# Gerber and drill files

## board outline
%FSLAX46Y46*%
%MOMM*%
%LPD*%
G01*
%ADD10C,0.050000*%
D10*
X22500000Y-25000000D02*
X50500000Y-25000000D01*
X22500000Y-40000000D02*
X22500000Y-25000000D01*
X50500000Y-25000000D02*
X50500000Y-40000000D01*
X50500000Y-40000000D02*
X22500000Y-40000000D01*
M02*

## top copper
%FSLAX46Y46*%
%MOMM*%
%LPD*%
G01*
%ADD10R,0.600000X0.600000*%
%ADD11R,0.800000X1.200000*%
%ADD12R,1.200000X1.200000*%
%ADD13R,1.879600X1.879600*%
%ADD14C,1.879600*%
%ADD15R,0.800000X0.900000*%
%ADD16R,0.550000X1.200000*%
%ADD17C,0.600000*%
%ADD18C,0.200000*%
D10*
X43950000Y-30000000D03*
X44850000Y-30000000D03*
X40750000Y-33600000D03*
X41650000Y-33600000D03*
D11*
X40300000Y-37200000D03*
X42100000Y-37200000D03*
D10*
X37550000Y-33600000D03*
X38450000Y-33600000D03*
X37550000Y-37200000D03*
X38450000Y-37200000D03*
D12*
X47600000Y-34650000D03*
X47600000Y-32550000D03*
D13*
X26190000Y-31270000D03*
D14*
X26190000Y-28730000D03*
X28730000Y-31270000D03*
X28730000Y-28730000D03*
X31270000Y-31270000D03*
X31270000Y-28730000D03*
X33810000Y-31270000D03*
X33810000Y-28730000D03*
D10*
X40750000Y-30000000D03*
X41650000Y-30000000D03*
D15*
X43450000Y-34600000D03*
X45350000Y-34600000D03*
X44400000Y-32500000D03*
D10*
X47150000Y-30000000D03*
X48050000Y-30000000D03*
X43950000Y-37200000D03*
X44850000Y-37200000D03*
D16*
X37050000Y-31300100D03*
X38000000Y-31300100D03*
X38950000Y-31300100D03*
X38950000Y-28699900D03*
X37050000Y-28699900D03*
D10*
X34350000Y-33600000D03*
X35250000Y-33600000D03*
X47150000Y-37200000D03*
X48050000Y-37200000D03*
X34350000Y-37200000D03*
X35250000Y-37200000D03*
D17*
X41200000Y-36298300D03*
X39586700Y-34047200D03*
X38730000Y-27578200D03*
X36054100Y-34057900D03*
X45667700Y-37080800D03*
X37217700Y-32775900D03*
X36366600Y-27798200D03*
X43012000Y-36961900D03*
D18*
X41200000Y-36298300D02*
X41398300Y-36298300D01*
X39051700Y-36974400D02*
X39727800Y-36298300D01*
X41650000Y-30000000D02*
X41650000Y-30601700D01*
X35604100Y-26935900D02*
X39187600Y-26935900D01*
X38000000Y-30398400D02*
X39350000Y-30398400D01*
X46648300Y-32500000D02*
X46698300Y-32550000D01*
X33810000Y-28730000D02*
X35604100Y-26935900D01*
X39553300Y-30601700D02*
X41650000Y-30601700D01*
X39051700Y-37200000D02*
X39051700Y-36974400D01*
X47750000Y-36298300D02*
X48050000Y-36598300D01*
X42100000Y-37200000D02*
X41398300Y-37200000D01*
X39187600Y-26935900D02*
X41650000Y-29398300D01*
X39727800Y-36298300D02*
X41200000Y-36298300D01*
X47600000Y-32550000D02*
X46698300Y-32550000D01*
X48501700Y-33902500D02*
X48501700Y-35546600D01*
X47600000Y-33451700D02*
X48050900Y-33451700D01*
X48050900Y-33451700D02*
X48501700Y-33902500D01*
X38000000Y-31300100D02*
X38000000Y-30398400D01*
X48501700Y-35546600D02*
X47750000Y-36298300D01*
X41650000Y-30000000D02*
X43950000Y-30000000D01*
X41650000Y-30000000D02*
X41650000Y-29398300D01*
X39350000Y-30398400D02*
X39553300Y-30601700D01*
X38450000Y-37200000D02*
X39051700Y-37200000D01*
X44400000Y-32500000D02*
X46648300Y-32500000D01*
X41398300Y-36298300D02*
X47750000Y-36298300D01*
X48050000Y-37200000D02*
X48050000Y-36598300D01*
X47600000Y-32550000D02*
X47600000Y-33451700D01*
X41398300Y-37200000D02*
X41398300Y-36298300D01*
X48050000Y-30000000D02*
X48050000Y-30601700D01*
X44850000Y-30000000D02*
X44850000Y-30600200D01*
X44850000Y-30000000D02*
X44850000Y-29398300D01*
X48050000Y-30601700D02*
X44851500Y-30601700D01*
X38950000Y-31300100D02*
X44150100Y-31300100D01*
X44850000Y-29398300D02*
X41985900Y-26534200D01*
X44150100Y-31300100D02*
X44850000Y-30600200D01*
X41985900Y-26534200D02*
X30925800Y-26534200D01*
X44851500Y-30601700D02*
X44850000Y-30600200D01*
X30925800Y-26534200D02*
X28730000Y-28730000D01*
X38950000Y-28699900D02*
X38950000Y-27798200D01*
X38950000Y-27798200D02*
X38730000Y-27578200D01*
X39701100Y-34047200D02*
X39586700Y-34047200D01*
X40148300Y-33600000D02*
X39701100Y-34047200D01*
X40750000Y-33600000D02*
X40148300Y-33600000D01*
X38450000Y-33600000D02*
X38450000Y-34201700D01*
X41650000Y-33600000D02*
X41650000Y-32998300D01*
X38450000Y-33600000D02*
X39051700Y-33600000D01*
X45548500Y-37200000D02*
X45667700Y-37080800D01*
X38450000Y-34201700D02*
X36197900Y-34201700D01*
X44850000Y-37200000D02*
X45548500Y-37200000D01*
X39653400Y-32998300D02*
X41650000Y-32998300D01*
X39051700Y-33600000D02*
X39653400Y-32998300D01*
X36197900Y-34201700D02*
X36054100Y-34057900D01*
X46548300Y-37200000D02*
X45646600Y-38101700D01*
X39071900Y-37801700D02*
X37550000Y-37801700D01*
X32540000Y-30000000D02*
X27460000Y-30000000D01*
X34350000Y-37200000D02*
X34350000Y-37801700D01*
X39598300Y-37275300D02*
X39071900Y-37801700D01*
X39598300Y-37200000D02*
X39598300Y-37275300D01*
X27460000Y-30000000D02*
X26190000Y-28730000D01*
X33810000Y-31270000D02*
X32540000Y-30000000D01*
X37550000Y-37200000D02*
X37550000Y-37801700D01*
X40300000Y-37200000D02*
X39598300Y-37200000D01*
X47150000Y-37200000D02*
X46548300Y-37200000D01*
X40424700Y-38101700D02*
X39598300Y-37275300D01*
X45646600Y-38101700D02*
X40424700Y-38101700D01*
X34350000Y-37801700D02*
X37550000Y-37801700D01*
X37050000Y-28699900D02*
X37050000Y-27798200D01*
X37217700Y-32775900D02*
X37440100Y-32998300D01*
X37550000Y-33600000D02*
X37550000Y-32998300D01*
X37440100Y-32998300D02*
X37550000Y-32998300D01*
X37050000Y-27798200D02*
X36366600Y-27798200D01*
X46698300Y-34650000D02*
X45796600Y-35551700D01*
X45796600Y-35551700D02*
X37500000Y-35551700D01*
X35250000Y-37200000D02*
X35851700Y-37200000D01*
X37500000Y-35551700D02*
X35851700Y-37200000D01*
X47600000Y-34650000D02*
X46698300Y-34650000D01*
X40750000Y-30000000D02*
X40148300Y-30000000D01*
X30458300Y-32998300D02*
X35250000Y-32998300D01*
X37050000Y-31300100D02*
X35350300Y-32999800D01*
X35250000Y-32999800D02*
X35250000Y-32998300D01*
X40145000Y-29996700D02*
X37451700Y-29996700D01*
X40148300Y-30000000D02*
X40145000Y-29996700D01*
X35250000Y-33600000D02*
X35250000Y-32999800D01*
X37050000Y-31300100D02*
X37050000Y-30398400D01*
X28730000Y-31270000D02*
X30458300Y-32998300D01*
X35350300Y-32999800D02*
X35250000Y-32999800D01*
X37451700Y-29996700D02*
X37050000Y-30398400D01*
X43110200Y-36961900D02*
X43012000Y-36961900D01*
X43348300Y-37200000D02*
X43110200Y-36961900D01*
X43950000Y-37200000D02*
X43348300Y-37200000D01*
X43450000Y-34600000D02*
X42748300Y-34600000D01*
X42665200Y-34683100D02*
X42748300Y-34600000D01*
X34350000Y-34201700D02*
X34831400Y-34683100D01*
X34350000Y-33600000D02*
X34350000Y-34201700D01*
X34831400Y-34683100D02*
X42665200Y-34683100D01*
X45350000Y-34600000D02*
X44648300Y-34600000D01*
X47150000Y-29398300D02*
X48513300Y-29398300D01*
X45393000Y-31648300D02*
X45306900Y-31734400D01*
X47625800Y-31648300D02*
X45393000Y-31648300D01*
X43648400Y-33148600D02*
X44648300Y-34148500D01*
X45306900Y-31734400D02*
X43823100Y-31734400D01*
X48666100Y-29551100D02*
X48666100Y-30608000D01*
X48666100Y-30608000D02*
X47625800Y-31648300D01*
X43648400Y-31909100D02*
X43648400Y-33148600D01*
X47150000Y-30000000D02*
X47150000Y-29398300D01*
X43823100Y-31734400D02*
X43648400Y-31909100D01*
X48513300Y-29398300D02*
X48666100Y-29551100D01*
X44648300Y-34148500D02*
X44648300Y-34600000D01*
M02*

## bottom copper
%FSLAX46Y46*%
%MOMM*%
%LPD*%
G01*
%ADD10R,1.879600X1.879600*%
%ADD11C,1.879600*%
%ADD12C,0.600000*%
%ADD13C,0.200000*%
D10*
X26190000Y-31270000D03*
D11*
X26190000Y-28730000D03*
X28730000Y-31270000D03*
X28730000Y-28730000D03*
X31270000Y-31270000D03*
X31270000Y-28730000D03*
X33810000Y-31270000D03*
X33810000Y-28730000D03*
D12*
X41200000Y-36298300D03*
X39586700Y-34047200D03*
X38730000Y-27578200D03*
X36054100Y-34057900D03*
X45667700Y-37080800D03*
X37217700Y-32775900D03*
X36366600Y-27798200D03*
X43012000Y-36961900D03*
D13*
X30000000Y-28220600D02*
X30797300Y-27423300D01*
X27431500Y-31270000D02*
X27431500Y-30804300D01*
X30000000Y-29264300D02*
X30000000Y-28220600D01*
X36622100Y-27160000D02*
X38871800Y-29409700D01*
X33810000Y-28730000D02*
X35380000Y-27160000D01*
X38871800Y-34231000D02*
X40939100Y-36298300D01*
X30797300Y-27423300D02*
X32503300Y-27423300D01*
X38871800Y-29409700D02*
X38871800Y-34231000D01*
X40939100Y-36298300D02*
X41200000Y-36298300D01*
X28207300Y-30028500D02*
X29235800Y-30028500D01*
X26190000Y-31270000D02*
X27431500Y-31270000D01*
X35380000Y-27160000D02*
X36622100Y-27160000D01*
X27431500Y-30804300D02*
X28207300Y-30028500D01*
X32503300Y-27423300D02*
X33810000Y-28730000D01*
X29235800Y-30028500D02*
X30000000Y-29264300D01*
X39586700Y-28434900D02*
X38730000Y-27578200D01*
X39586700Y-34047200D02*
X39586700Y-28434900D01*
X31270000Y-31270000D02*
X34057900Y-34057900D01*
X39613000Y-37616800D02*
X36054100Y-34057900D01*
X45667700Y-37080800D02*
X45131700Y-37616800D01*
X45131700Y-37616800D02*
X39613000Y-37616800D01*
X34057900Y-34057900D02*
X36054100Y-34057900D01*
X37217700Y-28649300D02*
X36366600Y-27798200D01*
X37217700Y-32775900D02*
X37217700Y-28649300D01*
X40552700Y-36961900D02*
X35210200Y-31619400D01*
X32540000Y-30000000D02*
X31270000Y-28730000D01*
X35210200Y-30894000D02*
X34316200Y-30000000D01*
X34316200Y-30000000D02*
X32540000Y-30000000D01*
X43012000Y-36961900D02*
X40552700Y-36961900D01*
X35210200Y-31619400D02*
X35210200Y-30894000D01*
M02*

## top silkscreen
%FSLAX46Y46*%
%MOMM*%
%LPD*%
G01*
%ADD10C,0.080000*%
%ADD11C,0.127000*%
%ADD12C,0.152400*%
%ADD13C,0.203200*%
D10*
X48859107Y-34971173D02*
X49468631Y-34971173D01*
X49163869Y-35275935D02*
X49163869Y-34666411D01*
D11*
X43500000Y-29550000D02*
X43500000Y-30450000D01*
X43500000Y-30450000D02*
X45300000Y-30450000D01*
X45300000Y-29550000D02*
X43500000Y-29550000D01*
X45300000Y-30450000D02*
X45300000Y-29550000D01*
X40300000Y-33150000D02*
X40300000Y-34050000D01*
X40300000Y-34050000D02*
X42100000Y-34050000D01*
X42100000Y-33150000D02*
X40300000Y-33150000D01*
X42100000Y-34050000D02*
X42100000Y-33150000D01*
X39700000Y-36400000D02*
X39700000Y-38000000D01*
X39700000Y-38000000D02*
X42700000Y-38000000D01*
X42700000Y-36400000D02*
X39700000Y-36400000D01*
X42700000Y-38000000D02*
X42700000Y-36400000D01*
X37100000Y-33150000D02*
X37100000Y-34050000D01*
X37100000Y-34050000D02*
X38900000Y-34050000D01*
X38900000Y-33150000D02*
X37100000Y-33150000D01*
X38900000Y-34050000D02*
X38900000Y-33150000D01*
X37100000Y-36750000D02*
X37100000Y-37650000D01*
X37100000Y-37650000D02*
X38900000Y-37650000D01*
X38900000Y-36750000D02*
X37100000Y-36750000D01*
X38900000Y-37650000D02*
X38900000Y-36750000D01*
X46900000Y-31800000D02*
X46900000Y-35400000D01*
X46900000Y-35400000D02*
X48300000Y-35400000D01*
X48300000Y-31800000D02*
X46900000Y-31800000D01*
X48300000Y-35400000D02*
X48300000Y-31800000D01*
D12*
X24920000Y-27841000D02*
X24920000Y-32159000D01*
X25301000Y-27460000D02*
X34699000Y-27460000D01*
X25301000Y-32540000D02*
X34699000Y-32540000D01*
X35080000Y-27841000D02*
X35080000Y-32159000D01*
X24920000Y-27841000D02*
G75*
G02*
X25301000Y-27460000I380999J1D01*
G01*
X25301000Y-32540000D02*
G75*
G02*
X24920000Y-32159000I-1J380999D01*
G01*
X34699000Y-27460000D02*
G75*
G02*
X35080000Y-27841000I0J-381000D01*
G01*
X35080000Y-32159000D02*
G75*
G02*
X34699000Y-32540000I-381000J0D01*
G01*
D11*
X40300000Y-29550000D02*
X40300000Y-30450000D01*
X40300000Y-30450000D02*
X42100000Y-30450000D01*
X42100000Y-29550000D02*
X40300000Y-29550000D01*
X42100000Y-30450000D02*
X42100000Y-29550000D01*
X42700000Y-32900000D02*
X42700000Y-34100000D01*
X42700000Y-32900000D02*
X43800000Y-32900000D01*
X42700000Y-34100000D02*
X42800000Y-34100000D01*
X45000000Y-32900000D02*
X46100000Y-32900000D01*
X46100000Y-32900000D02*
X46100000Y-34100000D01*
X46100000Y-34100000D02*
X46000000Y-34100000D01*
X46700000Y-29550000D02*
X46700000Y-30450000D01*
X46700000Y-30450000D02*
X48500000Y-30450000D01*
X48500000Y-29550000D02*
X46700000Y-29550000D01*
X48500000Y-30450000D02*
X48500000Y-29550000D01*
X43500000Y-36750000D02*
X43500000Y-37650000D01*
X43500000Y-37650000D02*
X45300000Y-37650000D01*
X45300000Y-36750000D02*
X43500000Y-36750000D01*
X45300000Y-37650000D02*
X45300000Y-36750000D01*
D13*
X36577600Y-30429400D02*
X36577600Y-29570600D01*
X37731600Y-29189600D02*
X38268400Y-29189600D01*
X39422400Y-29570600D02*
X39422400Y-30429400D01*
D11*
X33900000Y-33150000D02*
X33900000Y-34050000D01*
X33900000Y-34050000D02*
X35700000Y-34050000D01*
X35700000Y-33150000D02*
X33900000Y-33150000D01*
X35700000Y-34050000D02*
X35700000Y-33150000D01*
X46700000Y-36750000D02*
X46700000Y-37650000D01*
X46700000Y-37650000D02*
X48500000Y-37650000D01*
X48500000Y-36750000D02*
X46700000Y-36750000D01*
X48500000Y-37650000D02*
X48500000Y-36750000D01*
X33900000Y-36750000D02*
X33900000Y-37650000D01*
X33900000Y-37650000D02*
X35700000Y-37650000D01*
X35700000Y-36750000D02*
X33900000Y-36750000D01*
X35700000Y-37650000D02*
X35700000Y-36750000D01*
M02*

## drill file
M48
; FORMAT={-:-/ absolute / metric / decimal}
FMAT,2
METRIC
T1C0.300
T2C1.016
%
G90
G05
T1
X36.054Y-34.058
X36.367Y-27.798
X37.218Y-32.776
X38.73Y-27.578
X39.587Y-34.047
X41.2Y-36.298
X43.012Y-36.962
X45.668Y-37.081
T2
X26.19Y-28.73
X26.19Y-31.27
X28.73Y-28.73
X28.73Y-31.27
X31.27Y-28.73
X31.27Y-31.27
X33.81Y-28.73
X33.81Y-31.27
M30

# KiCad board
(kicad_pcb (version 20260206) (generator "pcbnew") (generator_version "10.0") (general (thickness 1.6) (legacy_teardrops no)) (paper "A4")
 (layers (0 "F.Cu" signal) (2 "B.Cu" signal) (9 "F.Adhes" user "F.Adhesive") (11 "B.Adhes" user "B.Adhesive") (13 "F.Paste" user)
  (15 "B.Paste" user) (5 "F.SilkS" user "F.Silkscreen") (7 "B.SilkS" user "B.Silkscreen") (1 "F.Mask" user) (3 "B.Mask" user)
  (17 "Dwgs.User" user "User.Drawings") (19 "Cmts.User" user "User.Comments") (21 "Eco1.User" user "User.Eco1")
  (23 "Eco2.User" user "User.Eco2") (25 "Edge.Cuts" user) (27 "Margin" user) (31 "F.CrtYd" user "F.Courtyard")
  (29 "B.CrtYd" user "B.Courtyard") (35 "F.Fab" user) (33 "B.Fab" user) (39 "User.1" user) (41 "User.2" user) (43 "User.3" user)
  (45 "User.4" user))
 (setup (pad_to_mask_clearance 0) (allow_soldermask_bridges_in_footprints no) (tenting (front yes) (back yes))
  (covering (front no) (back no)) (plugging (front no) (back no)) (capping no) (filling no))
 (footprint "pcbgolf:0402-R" (layer "F.Cu") (at 44.4 30)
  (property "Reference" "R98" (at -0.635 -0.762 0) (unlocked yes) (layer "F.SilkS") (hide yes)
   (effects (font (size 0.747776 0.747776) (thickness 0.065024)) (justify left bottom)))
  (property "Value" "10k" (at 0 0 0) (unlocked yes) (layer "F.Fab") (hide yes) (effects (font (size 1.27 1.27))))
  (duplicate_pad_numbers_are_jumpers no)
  (fp_line (start -0.9 -0.45) (end -0.9 0.45) (stroke (width 0.127) (type solid)) (layer "F.SilkS"))
  (fp_line (start -0.9 0.45) (end 0.9 0.45) (stroke (width 0.127) (type solid)) (layer "F.SilkS"))
  (fp_line (start 0.9 -0.45) (end -0.9 -0.45) (stroke (width 0.127) (type solid)) (layer "F.SilkS"))
  (fp_line (start 0.9 0.45) (end 0.9 -0.45) (stroke (width 0.127) (type solid)) (layer "F.SilkS"))
  (pad "1" smd rect (at -0.45 0) (size 0.6 0.6) (layers "F.Cu" "F.Mask" "F.Paste") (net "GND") (solder_mask_margin 0.0508)
   (solder_paste_margin 0) (thermal_bridge_angle 0))
  (pad "2" smd rect (at 0.45 0) (size 0.6 0.6) (layers "F.Cu" "F.Mask" "F.Paste") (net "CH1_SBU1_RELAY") (solder_mask_margin 0.0508)
   (solder_paste_margin 0) (thermal_bridge_angle 0)))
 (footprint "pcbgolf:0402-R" (layer "F.Cu") (at 41.2 33.6)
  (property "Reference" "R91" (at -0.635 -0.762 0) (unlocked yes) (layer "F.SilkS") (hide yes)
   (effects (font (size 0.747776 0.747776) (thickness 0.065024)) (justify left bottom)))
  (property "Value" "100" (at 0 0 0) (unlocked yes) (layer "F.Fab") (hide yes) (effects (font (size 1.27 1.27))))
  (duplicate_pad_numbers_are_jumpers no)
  (fp_line (start -0.9 -0.45) (end -0.9 0.45) (stroke (width 0.127) (type solid)) (layer "F.SilkS"))
  (fp_line (start -0.9 0.45) (end 0.9 0.45) (stroke (width 0.127) (type solid)) (layer "F.SilkS"))
  (fp_line (start 0.9 -0.45) (end -0.9 -0.45) (stroke (width 0.127) (type solid)) (layer "F.SilkS"))
  (fp_line (start 0.9 0.45) (end 0.9 -0.45) (stroke (width 0.127) (type solid)) (layer "F.SilkS"))
  (pad "1" smd rect (at -0.45 0) (size 0.6 0.6) (layers "F.Cu" "F.Mask" "F.Paste") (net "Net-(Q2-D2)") (solder_mask_margin 0.0508)
   (solder_paste_margin 0) (thermal_bridge_angle 0))
  (pad "2" smd rect (at 0.45 0) (size 0.6 0.6) (layers "F.Cu" "F.Mask" "F.Paste") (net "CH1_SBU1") (solder_mask_margin 0.0508)
   (solder_paste_margin 0) (thermal_bridge_angle 0)))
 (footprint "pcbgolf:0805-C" (layer "F.Cu") (at 41.2 37.2)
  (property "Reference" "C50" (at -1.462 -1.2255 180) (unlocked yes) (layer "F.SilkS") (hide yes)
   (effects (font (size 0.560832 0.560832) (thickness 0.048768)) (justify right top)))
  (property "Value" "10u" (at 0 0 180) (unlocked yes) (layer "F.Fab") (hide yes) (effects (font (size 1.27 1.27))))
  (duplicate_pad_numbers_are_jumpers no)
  (fp_line (start -1.5 -0.8) (end -1.5 0.8) (stroke (width 0.127) (type solid)) (layer "F.SilkS"))
  (fp_line (start -1.5 0.8) (end 1.5 0.8) (stroke (width 0.127) (type solid)) (layer "F.SilkS"))
  (fp_line (start 1.5 -0.8) (end -1.5 -0.8) (stroke (width 0.127) (type solid)) (layer "F.SilkS"))
  (fp_line (start 1.5 0.8) (end 1.5 -0.8) (stroke (width 0.127) (type solid)) (layer "F.SilkS"))
  (pad "1" smd rect (at -0.9 0) (size 0.8 1.2) (layers "F.Cu" "F.Mask" "F.Paste") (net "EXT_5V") (solder_mask_margin 0.0508)
   (solder_paste_margin 0) (thermal_bridge_angle 0))
  (pad "2" smd rect (at 0.9 0) (size 0.8 1.2) (layers "F.Cu" "F.Mask" "F.Paste") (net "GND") (solder_mask_margin 0.0508)
   (solder_paste_margin 0) (thermal_bridge_angle 0)))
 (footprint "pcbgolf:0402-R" (layer "F.Cu") (at 38 33.6)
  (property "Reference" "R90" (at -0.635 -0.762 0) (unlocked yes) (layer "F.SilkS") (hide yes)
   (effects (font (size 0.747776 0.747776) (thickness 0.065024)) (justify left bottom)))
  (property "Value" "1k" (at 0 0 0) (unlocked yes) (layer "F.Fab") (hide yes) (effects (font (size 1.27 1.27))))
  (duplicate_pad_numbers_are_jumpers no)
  (fp_line (start -0.9 -0.45) (end -0.9 0.45) (stroke (width 0.127) (type solid)) (layer "F.SilkS"))
  (fp_line (start -0.9 0.45) (end 0.9 0.45) (stroke (width 0.127) (type solid)) (layer "F.SilkS"))
  (fp_line (start 0.9 -0.45) (end -0.9 -0.45) (stroke (width 0.127) (type solid)) (layer "F.SilkS"))
  (fp_line (start 0.9 0.45) (end 0.9 -0.45) (stroke (width 0.127) (type solid)) (layer "F.SilkS"))
  (pad "1" smd rect (at -0.45 0) (size 0.6 0.6) (layers "F.Cu" "F.Mask" "F.Paste") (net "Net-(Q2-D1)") (solder_mask_margin 0.0508)
   (solder_paste_margin 0) (thermal_bridge_angle 0))
  (pad "2" smd rect (at 0.45 0) (size 0.6 0.6) (layers "F.Cu" "F.Mask" "F.Paste") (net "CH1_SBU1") (solder_mask_margin 0.0508)
   (solder_paste_margin 0) (thermal_bridge_angle 0)))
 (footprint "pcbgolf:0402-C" (layer "F.Cu") (at 38 37.2)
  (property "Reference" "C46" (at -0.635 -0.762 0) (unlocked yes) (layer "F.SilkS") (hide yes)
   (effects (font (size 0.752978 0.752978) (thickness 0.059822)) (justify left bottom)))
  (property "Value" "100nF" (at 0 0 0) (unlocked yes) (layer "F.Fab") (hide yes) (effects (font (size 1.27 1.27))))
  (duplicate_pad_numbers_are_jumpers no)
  (fp_line (start -0.9 -0.45) (end -0.9 0.45) (stroke (width 0.127) (type solid)) (layer "F.SilkS"))
  (fp_line (start -0.9 0.45) (end 0.9 0.45) (stroke (width 0.127) (type solid)) (layer "F.SilkS"))
  (fp_line (start 0.9 -0.45) (end -0.9 -0.45) (stroke (width 0.127) (type solid)) (layer "F.SilkS"))
  (fp_line (start 0.9 0.45) (end 0.9 -0.45) (stroke (width 0.127) (type solid)) (layer "F.SilkS"))
  (pad "1" smd rect (at -0.45 0) (size 0.6 0.6) (layers "F.Cu" "F.Mask" "F.Paste") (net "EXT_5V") (solder_mask_margin 0.0508)
   (solder_paste_margin 0) (thermal_bridge_angle 0))
  (pad "2" smd rect (at 0.45 0) (size 0.6 0.6) (layers "F.Cu" "F.Mask" "F.Paste") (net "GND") (solder_mask_margin 0.0508)
   (solder_paste_margin 0) (thermal_bridge_angle 0)))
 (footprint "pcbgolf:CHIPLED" (layer "F.Cu") (at 47.6 33.6)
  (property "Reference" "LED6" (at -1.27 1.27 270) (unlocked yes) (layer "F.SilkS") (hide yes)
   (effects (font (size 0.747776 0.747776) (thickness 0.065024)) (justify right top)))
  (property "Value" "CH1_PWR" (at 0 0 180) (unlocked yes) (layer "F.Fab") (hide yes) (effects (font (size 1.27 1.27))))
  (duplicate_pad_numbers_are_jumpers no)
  (fp_line (start -0.7 -1.8) (end -0.7 1.8) (stroke (width 0.127) (type solid)) (layer "F.SilkS"))
  (fp_line (start -0.7 1.8) (end 0.7 1.8) (stroke (width 0.127) (type solid)) (layer "F.SilkS"))
  (fp_line (start 0.7 -1.8) (end -0.7 -1.8) (stroke (width 0.127) (type solid)) (layer "F.SilkS"))
  (fp_line (start 0.7 1.8) (end 0.7 -1.8) (stroke (width 0.127) (type solid)) (layer "F.SilkS"))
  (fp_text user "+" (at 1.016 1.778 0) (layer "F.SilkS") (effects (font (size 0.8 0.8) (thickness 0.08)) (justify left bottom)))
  (pad "A" smd rect (at 0 1.05) (size 1.2 1.2) (layers "F.Cu" "F.Mask" "F.Paste") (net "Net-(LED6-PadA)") (solder_mask_margin 0.0508)
   (solder_paste_margin 0) (thermal_bridge_angle 0))
  (pad "C" smd rect (at 0 -1.05) (size 1.2 1.2) (layers "F.Cu" "F.Mask" "F.Paste") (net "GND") (solder_mask_margin 0.0508)
   (solder_paste_margin 0) (thermal_bridge_angle 0)))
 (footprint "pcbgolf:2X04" (layer "F.Cu") (at 30 30)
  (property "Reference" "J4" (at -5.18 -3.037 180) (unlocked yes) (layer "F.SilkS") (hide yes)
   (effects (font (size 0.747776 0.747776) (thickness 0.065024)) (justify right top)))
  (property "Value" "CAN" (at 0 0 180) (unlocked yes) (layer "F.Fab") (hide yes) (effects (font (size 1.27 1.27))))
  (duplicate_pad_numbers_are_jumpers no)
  (fp_line (start -5.08 -2.159) (end -5.08 2.159) (stroke (width 0.1524) (type solid)) (layer "F.SilkS"))
  (fp_line (start -4.699 -2.54) (end 4.699 -2.54) (stroke (width 0.1524) (type solid)) (layer "F.SilkS"))
  (fp_line (start -4.699 2.54) (end 4.699 2.54) (stroke (width 0.1524) (type solid)) (layer "F.SilkS"))
  (fp_line (start 5.08 -2.159) (end 5.08 2.159) (stroke (width 0.1524) (type solid)) (layer "F.SilkS"))
  (fp_arc (start -5.08 -2.159) (mid -4.968408 -2.428408) (end -4.699 -2.54) (stroke (width 0.1524) (type solid)) (layer "F.SilkS"))
  (fp_arc (start -4.699 2.54) (mid -4.968408 2.428408) (end -5.08 2.159) (stroke (width 0.1524) (type solid)) (layer "F.SilkS"))
  (fp_arc (start 4.699 -2.54) (mid 4.968408 -2.428408) (end 5.08 -2.159) (stroke (width 0.1524) (type solid)) (layer "F.SilkS"))
  (fp_arc (start 5.08 2.159) (mid 4.968408 2.428408) (end 4.699 2.54) (stroke (width 0.1524) (type solid)) (layer "F.SilkS"))
  (pad "1" thru_hole rect (at -3.81 1.27 90) (size 1.8796 1.8796) (drill 1.016) (layers "*.Cu" "*.Mask") (remove_unused_layers no)
   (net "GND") (solder_mask_margin 0.0508) (thermal_bridge_angle 0))
  (pad "2" thru_hole circle (at -3.81 -1.27 90) (size 1.8796 1.8796) (drill 1.016) (layers "*.Cu" "*.Mask") (remove_unused_layers no)
   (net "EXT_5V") (solder_mask_margin 0.0508) (thermal_bridge_angle 0))
  (pad "3" thru_hole circle (at -1.27 1.27 90) (size 1.8796 1.8796) (drill 1.016) (layers "*.Cu" "*.Mask") (remove_unused_layers no)
   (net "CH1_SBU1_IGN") (solder_mask_margin 0.0508) (thermal_bridge_angle 0))
  (pad "4" thru_hole circle (at -1.27 -1.27 90) (size 1.8796 1.8796) (drill 1.016) (layers "*.Cu" "*.Mask") (remove_unused_layers no)
   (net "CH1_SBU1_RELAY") (solder_mask_margin 0.0508) (thermal_bridge_angle 0))
  (pad "5" thru_hole circle (at 1.27 1.27 90) (size 1.8796 1.8796) (drill 1.016) (layers "*.Cu" "*.Mask") (remove_unused_layers no)
   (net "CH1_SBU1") (solder_mask_margin 0.0508) (thermal_bridge_angle 0))
  (pad "6" thru_hole circle (at 1.27 -1.27 90) (size 1.8796 1.8796) (drill 1.016) (layers "*.Cu" "*.Mask") (remove_unused_layers no)
   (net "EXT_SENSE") (solder_mask_margin 0.0508) (thermal_bridge_angle 0))
  (pad "7" thru_hole circle (at 3.81 1.27 90) (size 1.8796 1.8796) (drill 1.016) (layers "*.Cu" "*.Mask") (remove_unused_layers no)
   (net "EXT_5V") (solder_mask_margin 0.0508) (thermal_bridge_angle 0))
  (pad "8" thru_hole circle (at 3.81 -1.27 90) (size 1.8796 1.8796) (drill 1.016) (layers "*.Cu" "*.Mask") (remove_unused_layers no)
   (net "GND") (solder_mask_margin 0.0508) (thermal_bridge_angle 0)))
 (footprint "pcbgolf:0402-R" (layer "F.Cu") (at 41.2 30)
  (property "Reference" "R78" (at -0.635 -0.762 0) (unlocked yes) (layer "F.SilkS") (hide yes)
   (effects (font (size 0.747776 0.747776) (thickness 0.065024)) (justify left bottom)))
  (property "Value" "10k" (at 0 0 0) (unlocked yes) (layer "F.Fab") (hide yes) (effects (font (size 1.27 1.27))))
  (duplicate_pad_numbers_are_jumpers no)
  (fp_line (start -0.9 -0.45) (end -0.9 0.45) (stroke (width 0.127) (type solid)) (layer "F.SilkS"))
  (fp_line (start -0.9 0.45) (end 0.9 0.45) (stroke (width 0.127) (type solid)) (layer "F.SilkS"))
  (fp_line (start 0.9 -0.45) (end -0.9 -0.45) (stroke (width 0.127) (type solid)) (layer "F.SilkS"))
  (fp_line (start 0.9 0.45) (end 0.9 -0.45) (stroke (width 0.127) (type solid)) (layer "F.SilkS"))
  (pad "1" smd rect (at -0.45 0) (size 0.6 0.6) (layers "F.Cu" "F.Mask" "F.Paste") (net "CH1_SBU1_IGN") (solder_mask_margin 0.0508)
   (solder_paste_margin 0) (thermal_bridge_angle 0))
  (pad "2" smd rect (at 0.45 0) (size 0.6 0.6) (layers "F.Cu" "F.Mask" "F.Paste") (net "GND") (solder_mask_margin 0.0508)
   (solder_paste_margin 0) (thermal_bridge_angle 0)))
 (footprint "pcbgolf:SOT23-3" (layer "F.Cu") (at 44.4 33.6)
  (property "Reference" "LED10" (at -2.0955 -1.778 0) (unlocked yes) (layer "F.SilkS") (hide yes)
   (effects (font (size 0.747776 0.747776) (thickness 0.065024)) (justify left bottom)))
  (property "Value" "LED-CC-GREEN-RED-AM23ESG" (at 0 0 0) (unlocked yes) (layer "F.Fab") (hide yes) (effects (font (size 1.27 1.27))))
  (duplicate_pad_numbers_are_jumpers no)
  (fp_line (start -1.7 -0.7) (end -1.7 0.5) (stroke (width 0.127) (type solid)) (layer "F.SilkS"))
  (fp_line (start -1.7 -0.7) (end -0.6 -0.7) (stroke (width 0.127) (type solid)) (layer "F.SilkS"))
  (fp_line (start -1.7 0.5) (end -1.6 0.5) (stroke (width 0.127) (type solid)) (layer "F.SilkS"))
  (fp_line (start 0.6 -0.7) (end 1.7 -0.7) (stroke (width 0.127) (type solid)) (layer "F.SilkS"))
  (fp_line (start 1.7 -0.7) (end 1.7 0.5) (stroke (width 0.127) (type solid)) (layer "F.SilkS"))
  (fp_line (start 1.7 0.5) (end 1.6 0.5) (stroke (width 0.127) (type solid)) (layer "F.SilkS"))
  (pad "1" smd rect (at -0.95 1) (size 0.8 0.9) (layers "F.Cu" "F.Mask" "F.Paste") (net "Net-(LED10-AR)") (solder_mask_margin 0.0508)
   (solder_paste_margin 0) (thermal_bridge_angle 0))
  (pad "2" smd rect (at 0.95 1) (size 0.8 0.9) (layers "F.Cu" "F.Mask" "F.Paste") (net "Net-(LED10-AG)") (solder_mask_margin 0.0508)
   (solder_paste_margin 0) (thermal_bridge_angle 0))
  (pad "3" smd rect (at 0 -1.1) (size 0.8 0.9) (layers "F.Cu" "F.Mask" "F.Paste") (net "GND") (solder_mask_margin 0.0508)
   (solder_paste_margin 0) (thermal_bridge_angle 0)))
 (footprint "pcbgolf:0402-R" (layer "F.Cu") (at 47.6 30)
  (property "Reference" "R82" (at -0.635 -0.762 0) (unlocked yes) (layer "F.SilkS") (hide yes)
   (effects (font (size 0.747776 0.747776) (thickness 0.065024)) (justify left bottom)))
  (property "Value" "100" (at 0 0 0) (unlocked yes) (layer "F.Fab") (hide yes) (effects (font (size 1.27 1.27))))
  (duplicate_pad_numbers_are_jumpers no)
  (fp_line (start -0.9 -0.45) (end -0.9 0.45) (stroke (width 0.127) (type solid)) (layer "F.SilkS"))
  (fp_line (start -0.9 0.45) (end 0.9 0.45) (stroke (width 0.127) (type solid)) (layer "F.SilkS"))
  (fp_line (start 0.9 -0.45) (end -0.9 -0.45) (stroke (width 0.127) (type solid)) (layer "F.SilkS"))
  (fp_line (start 0.9 0.45) (end 0.9 -0.45) (stroke (width 0.127) (type solid)) (layer "F.SilkS"))
  (pad "1" smd rect (at -0.45 0) (size 0.6 0.6) (layers "F.Cu" "F.Mask" "F.Paste") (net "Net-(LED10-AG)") (solder_mask_margin 0.0508)
   (solder_paste_margin 0) (thermal_bridge_angle 0))
  (pad "2" smd rect (at 0.45 0) (size 0.6 0.6) (layers "F.Cu" "F.Mask" "F.Paste") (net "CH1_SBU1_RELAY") (solder_mask_margin 0.0508)
   (solder_paste_margin 0) (thermal_bridge_angle 0)))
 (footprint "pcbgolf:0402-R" (layer "F.Cu") (at 44.4 37.2)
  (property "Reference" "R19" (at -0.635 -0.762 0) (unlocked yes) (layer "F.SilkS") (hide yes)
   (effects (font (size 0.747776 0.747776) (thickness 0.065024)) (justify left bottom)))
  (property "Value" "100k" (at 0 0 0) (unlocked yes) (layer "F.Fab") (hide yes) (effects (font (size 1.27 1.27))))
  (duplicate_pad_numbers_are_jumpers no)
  (fp_line (start -0.9 -0.45) (end -0.9 0.45) (stroke (width 0.127) (type solid)) (layer "F.SilkS"))
  (fp_line (start -0.9 0.45) (end 0.9 0.45) (stroke (width 0.127) (type solid)) (layer "F.SilkS"))
  (fp_line (start 0.9 -0.45) (end -0.9 -0.45) (stroke (width 0.127) (type solid)) (layer "F.SilkS"))
  (fp_line (start 0.9 0.45) (end 0.9 -0.45) (stroke (width 0.127) (type solid)) (layer "F.SilkS"))
  (pad "1" smd rect (at -0.45 0) (size 0.6 0.6) (layers "F.Cu" "F.Mask" "F.Paste") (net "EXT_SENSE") (solder_mask_margin 0.0508)
   (solder_paste_margin 0) (thermal_bridge_angle 0))
  (pad "2" smd rect (at 0.45 0) (size 0.6 0.6) (layers "F.Cu" "F.Mask" "F.Paste") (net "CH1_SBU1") (solder_mask_margin 0.0508)
   (solder_paste_margin 0) (thermal_bridge_angle 0)))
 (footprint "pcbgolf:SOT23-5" (layer "F.Cu") (at 38 30)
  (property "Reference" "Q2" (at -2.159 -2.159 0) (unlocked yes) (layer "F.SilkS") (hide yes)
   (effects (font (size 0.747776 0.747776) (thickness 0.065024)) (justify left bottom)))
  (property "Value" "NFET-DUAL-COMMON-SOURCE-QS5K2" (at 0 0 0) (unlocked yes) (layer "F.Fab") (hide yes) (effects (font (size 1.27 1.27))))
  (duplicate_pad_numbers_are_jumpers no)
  (fp_line (start -1.4224 0.4294) (end -1.4224 -0.4294) (stroke (width 0.2032) (type solid)) (layer "F.SilkS"))
  (fp_line (start -0.2684 -0.8104) (end 0.2684 -0.8104) (stroke (width 0.2032) (type solid)) (layer "F.SilkS"))
  (fp_line (start 1.4224 -0.4294) (end 1.4224 0.4294) (stroke (width 0.2032) (type solid)) (layer "F.SilkS"))
  (pad "1" smd rect (at -0.95 1.3001) (size 0.55 1.2) (layers "F.Cu" "F.Mask" "F.Paste") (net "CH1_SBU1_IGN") (solder_mask_margin 0.0508)
   (solder_paste_margin 0) (thermal_bridge_angle 0))
  (pad "2" smd rect (at 0 1.3001) (size 0.55 1.2) (layers "F.Cu" "F.Mask" "F.Paste") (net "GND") (solder_mask_margin 0.0508)
   (solder_paste_margin 0) (thermal_bridge_angle 0))
  (pad "3" smd rect (at 0.95 1.3001) (size 0.55 1.2) (layers "F.Cu" "F.Mask" "F.Paste") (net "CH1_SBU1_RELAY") (solder_mask_margin 0.0508)
   (solder_paste_margin 0) (thermal_bridge_angle 0))
  (pad "4" smd rect (at 0.95 -1.3001) (size 0.55 1.2) (layers "F.Cu" "F.Mask" "F.Paste") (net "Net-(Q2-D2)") (solder_mask_margin 0.0508)
   (solder_paste_margin 0) (thermal_bridge_angle 0))
  (pad "5" smd rect (at -0.95 -1.3001) (size 0.55 1.2) (layers "F.Cu" "F.Mask" "F.Paste") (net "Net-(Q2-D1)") (solder_mask_margin 0.0508)
   (solder_paste_margin 0) (thermal_bridge_angle 0)))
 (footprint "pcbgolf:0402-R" (layer "F.Cu") (at 34.8 33.6)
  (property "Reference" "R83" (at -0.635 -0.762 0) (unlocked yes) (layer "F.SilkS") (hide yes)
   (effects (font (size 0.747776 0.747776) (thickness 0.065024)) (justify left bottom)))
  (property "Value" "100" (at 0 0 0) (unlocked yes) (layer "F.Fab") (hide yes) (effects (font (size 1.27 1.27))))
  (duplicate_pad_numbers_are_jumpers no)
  (fp_line (start -0.9 -0.45) (end -0.9 0.45) (stroke (width 0.127) (type solid)) (layer "F.SilkS"))
  (fp_line (start -0.9 0.45) (end 0.9 0.45) (stroke (width 0.127) (type solid)) (layer "F.SilkS"))
  (fp_line (start 0.9 -0.45) (end -0.9 -0.45) (stroke (width 0.127) (type solid)) (layer "F.SilkS"))
  (fp_line (start 0.9 0.45) (end 0.9 -0.45) (stroke (width 0.127) (type solid)) (layer "F.SilkS"))
  (pad "1" smd rect (at -0.45 0) (size 0.6 0.6) (layers "F.Cu" "F.Mask" "F.Paste") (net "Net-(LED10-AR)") (solder_mask_margin 0.0508)
   (solder_paste_margin 0) (thermal_bridge_angle 0))
  (pad "2" smd rect (at 0.45 0) (size 0.6 0.6) (layers "F.Cu" "F.Mask" "F.Paste") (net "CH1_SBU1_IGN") (solder_mask_margin 0.0508)
   (solder_paste_margin 0) (thermal_bridge_angle 0)))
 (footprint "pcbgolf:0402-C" (layer "F.Cu") (at 47.6 37.2)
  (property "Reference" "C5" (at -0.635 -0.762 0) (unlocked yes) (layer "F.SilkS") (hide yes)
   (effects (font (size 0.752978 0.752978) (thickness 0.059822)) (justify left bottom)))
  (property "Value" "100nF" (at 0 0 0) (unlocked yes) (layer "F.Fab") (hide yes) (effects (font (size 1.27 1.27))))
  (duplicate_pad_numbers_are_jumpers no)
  (fp_line (start -0.9 -0.45) (end -0.9 0.45) (stroke (width 0.127) (type solid)) (layer "F.SilkS"))
  (fp_line (start -0.9 0.45) (end 0.9 0.45) (stroke (width 0.127) (type solid)) (layer "F.SilkS"))
  (fp_line (start 0.9 -0.45) (end -0.9 -0.45) (stroke (width 0.127) (type solid)) (layer "F.SilkS"))
  (fp_line (start 0.9 0.45) (end 0.9 -0.45) (stroke (width 0.127) (type solid)) (layer "F.SilkS"))
  (pad "1" smd rect (at -0.45 0) (size 0.6 0.6) (layers "F.Cu" "F.Mask" "F.Paste") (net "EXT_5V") (solder_mask_margin 0.0508)
   (solder_paste_margin 0) (thermal_bridge_angle 0))
  (pad "2" smd rect (at 0.45 0) (size 0.6 0.6) (layers "F.Cu" "F.Mask" "F.Paste") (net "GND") (solder_mask_margin 0.0508)
   (solder_paste_margin 0) (thermal_bridge_angle 0)))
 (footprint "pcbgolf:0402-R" (layer "F.Cu") (at 34.8 37.2)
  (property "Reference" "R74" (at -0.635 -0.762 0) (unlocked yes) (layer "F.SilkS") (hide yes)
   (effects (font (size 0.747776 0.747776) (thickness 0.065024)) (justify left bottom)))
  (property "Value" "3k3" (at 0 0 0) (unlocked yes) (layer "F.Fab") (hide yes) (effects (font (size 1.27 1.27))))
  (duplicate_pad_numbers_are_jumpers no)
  (fp_line (start -0.9 -0.45) (end -0.9 0.45) (stroke (width 0.127) (type solid)) (layer "F.SilkS"))
  (fp_line (start -0.9 0.45) (end 0.9 0.45) (stroke (width 0.127) (type solid)) (layer "F.SilkS"))
  (fp_line (start 0.9 -0.45) (end -0.9 -0.45) (stroke (width 0.127) (type solid)) (layer "F.SilkS"))
  (fp_line (start 0.9 0.45) (end 0.9 -0.45) (stroke (width 0.127) (type solid)) (layer "F.SilkS"))
  (pad "1" smd rect (at -0.45 0) (size 0.6 0.6) (layers "F.Cu" "F.Mask" "F.Paste") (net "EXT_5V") (solder_mask_margin 0.0508)
   (solder_paste_margin 0) (thermal_bridge_angle 0))
  (pad "2" smd rect (at 0.45 0) (size 0.6 0.6) (layers "F.Cu" "F.Mask" "F.Paste") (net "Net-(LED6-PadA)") (solder_mask_margin 0.0508)
   (solder_paste_margin 0) (thermal_bridge_angle 0)))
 (gr_line (start 22.5 25) (end 50.5 25) (stroke (width 0.05) (type default)) (layer "Edge.Cuts"))
 (gr_line (start 22.5 40) (end 22.5 25) (stroke (width 0.05) (type default)) (layer "Edge.Cuts"))
 (gr_line (start 50.5 25) (end 50.5 40) (stroke (width 0.05) (type default)) (layer "Edge.Cuts"))
 (gr_line (start 50.5 40) (end 22.5 40) (stroke (width 0.05) (type default)) (layer "Edge.Cuts"))
 (segment (start 41.2 36.2983) (end 41.3983 36.2983) (width 0.2) (layer "F.Cu") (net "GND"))
 (segment (start 39.0517 36.9744) (end 39.7278 36.2983) (width 0.2) (layer "F.Cu") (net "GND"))
 (segment (start 41.65 30) (end 41.65 30.6017) (width 0.2) (layer "F.Cu") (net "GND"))
 (segment (start 35.6041 26.9359) (end 39.1876 26.9359) (width 0.2) (layer "F.Cu") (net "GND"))
 (segment (start 38 30.3984) (end 39.35 30.3984) (width 0.2) (layer "F.Cu") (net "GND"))
 (segment (start 46.6483 32.5) (end 46.6983 32.55) (width 0.2) (layer "F.Cu") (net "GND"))
 (segment (start 33.81 28.73) (end 35.6041 26.9359) (width 0.2) (layer "F.Cu") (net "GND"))
 (segment (start 39.5533 30.6017) (end 41.65 30.6017) (width 0.2) (layer "F.Cu") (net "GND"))
 (segment (start 39.0517 37.2) (end 39.0517 36.9744) (width 0.2) (layer "F.Cu") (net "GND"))
 (segment (start 47.75 36.2983) (end 48.05 36.5983) (width 0.2) (layer "F.Cu") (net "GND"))
 (segment (start 42.1 37.2) (end 41.3983 37.2) (width 0.2) (layer "F.Cu") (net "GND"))
 (segment (start 39.1876 26.9359) (end 41.65 29.3983) (width 0.2) (layer "F.Cu") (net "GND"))
 (segment (start 39.7278 36.2983) (end 41.2 36.2983) (width 0.2) (layer "F.Cu") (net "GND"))
 (segment (start 47.6 32.55) (end 46.6983 32.55) (width 0.2) (layer "F.Cu") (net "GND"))
 (segment (start 48.5017 33.9025) (end 48.5017 35.5466) (width 0.2) (layer "F.Cu") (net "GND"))
 (segment (start 47.6 33.4517) (end 48.0509 33.4517) (width 0.2) (layer "F.Cu") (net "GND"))
 (segment (start 48.0509 33.4517) (end 48.5017 33.9025) (width 0.2) (layer "F.Cu") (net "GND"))
 (segment (start 38 31.3001) (end 38 30.3984) (width 0.2) (layer "F.Cu") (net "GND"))
 (segment (start 48.5017 35.5466) (end 47.75 36.2983) (width 0.2) (layer "F.Cu") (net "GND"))
 (segment (start 41.65 30) (end 43.95 30) (width 0.2) (layer "F.Cu") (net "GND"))
 (segment (start 41.65 30) (end 41.65 29.3983) (width 0.2) (layer "F.Cu") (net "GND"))
 (segment (start 39.35 30.3984) (end 39.5533 30.6017) (width 0.2) (layer "F.Cu") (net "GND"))
 (segment (start 38.45 37.2) (end 39.0517 37.2) (width 0.2) (layer "F.Cu") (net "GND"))
 (segment (start 44.4 32.5) (end 46.6483 32.5) (width 0.2) (layer "F.Cu") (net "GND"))
 (segment (start 41.3983 36.2983) (end 47.75 36.2983) (width 0.2) (layer "F.Cu") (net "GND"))
 (segment (start 48.05 37.2) (end 48.05 36.5983) (width 0.2) (layer "F.Cu") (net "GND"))
 (segment (start 47.6 32.55) (end 47.6 33.4517) (width 0.2) (layer "F.Cu") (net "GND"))
 (segment (start 41.3983 37.2) (end 41.3983 36.2983) (width 0.2) (layer "F.Cu") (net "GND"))
 (via (at 41.2 36.2983) (size 0.6) (drill 0.3) (layers "F.Cu" "B.Cu") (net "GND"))
 (segment (start 30 28.2206) (end 30.7973 27.4233) (width 0.2) (layer "B.Cu") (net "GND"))
 (segment (start 27.4315 31.27) (end 27.4315 30.8043) (width 0.2) (layer "B.Cu") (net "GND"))
 (segment (start 30 29.2643) (end 30 28.2206) (width 0.2) (layer "B.Cu") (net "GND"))
 (segment (start 36.6221 27.16) (end 38.8718 29.4097) (width 0.2) (layer "B.Cu") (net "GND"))
 (segment (start 33.81 28.73) (end 35.38 27.16) (width 0.2) (layer "B.Cu") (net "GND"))
 (segment (start 38.8718 34.231) (end 40.9391 36.2983) (width 0.2) (layer "B.Cu") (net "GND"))
 (segment (start 30.7973 27.4233) (end 32.5033 27.4233) (width 0.2) (layer "B.Cu") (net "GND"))
 (segment (start 38.8718 29.4097) (end 38.8718 34.231) (width 0.2) (layer "B.Cu") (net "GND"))
 (segment (start 40.9391 36.2983) (end 41.2 36.2983) (width 0.2) (layer "B.Cu") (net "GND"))
 (segment (start 28.2073 30.0285) (end 29.2358 30.0285) (width 0.2) (layer "B.Cu") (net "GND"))
 (segment (start 26.19 31.27) (end 27.4315 31.27) (width 0.2) (layer "B.Cu") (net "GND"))
 (segment (start 35.38 27.16) (end 36.6221 27.16) (width 0.2) (layer "B.Cu") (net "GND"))
 (segment (start 27.4315 30.8043) (end 28.2073 30.0285) (width 0.2) (layer "B.Cu") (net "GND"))
 (segment (start 32.5033 27.4233) (end 33.81 28.73) (width 0.2) (layer "B.Cu") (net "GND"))
 (segment (start 29.2358 30.0285) (end 30 29.2643) (width 0.2) (layer "B.Cu") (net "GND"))
 (segment (start 48.05 30) (end 48.05 30.6017) (width 0.2) (layer "F.Cu") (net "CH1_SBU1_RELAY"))
 (segment (start 44.85 30) (end 44.85 30.6002) (width 0.2) (layer "F.Cu") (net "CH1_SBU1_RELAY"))
 (segment (start 44.85 30) (end 44.85 29.3983) (width 0.2) (layer "F.Cu") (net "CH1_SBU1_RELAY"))
 (segment (start 48.05 30.6017) (end 44.8515 30.6017) (width 0.2) (layer "F.Cu") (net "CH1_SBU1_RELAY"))
 (segment (start 38.95 31.3001) (end 44.1501 31.3001) (width 0.2) (layer "F.Cu") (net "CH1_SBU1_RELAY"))
 (segment (start 44.85 29.3983) (end 41.9859 26.5342) (width 0.2) (layer "F.Cu") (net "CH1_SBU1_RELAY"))
 (segment (start 44.1501 31.3001) (end 44.85 30.6002) (width 0.2) (layer "F.Cu") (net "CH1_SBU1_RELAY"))
 (segment (start 41.9859 26.5342) (end 30.9258 26.5342) (width 0.2) (layer "F.Cu") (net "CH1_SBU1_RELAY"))
 (segment (start 44.8515 30.6017) (end 44.85 30.6002) (width 0.2) (layer "F.Cu") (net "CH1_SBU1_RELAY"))
 (segment (start 30.9258 26.5342) (end 28.73 28.73) (width 0.2) (layer "F.Cu") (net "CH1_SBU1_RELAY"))
 (segment (start 38.95 28.6999) (end 38.95 27.7982) (width 0.2) (layer "F.Cu") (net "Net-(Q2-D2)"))
 (segment (start 38.95 27.7982) (end 38.73 27.5782) (width 0.2) (layer "F.Cu") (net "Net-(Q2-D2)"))
 (segment (start 39.7011 34.0472) (end 39.5867 34.0472) (width 0.2) (layer "F.Cu") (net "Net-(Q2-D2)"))
 (segment (start 40.1483 33.6) (end 39.7011 34.0472) (width 0.2) (layer "F.Cu") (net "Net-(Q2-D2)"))
 (segment (start 40.75 33.6) (end 40.1483 33.6) (width 0.2) (layer "F.Cu") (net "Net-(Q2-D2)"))
 (via (at 39.5867 34.0472) (size 0.6) (drill 0.3) (layers "F.Cu" "B.Cu") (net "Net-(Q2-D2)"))
 (via (at 38.73 27.5782) (size 0.6) (drill 0.3) (layers "F.Cu" "B.Cu") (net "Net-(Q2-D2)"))
 (segment (start 39.5867 28.4349) (end 38.73 27.5782) (width 0.2) (layer "B.Cu") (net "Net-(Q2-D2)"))
 (segment (start 39.5867 34.0472) (end 39.5867 28.4349) (width 0.2) (layer "B.Cu") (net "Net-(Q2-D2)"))
 (segment (start 38.45 33.6) (end 38.45 34.2017) (width 0.2) (layer "F.Cu") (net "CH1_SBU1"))
 (segment (start 41.65 33.6) (end 41.65 32.9983) (width 0.2) (layer "F.Cu") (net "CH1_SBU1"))
 (segment (start 38.45 33.6) (end 39.0517 33.6) (width 0.2) (layer "F.Cu") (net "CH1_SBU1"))
 (segment (start 45.5485 37.2) (end 45.6677 37.0808) (width 0.2) (layer "F.Cu") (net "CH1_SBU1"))
 (segment (start 38.45 34.2017) (end 36.1979 34.2017) (width 0.2) (layer "F.Cu") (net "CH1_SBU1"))
 (segment (start 44.85 37.2) (end 45.5485 37.2) (width 0.2) (layer "F.Cu") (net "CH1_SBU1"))
 (segment (start 39.6534 32.9983) (end 41.65 32.9983) (width 0.2) (layer "F.Cu") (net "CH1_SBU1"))
 (segment (start 39.0517 33.6) (end 39.6534 32.9983) (width 0.2) (layer "F.Cu") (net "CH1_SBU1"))
 (segment (start 36.1979 34.2017) (end 36.0541 34.0579) (width 0.2) (layer "F.Cu") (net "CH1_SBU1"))
 (via (at 36.0541 34.0579) (size 0.6) (drill 0.3) (layers "F.Cu" "B.Cu") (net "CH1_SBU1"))
 (via (at 45.6677 37.0808) (size 0.6) (drill 0.3) (layers "F.Cu" "B.Cu") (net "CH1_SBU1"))
 (segment (start 31.27 31.27) (end 34.0579 34.0579) (width 0.2) (layer "B.Cu") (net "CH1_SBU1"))
 (segment (start 39.613 37.6168) (end 36.0541 34.0579) (width 0.2) (layer "B.Cu") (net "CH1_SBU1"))
 (segment (start 45.6677 37.0808) (end 45.1317 37.6168) (width 0.2) (layer "B.Cu") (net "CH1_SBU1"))
 (segment (start 45.1317 37.6168) (end 39.613 37.6168) (width 0.2) (layer "B.Cu") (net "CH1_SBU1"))
 (segment (start 34.0579 34.0579) (end 36.0541 34.0579) (width 0.2) (layer "B.Cu") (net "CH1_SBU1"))
 (segment (start 46.5483 37.2) (end 45.6466 38.1017) (width 0.2) (layer "F.Cu") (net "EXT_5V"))
 (segment (start 39.0719 37.8017) (end 37.55 37.8017) (width 0.2) (layer "F.Cu") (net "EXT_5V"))
 (segment (start 32.54 30) (end 27.46 30) (width 0.2) (layer "F.Cu") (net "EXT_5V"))
 (segment (start 34.35 37.2) (end 34.35 37.8017) (width 0.2) (layer "F.Cu") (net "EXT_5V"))
 (segment (start 39.5983 37.2753) (end 39.0719 37.8017) (width 0.2) (layer "F.Cu") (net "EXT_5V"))
 (segment (start 39.5983 37.2) (end 39.5983 37.2753) (width 0.2) (layer "F.Cu") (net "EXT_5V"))
 (segment (start 27.46 30) (end 26.19 28.73) (width 0.2) (layer "F.Cu") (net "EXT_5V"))
 (segment (start 33.81 31.27) (end 32.54 30) (width 0.2) (layer "F.Cu") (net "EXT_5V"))
 (segment (start 37.55 37.2) (end 37.55 37.8017) (width 0.2) (layer "F.Cu") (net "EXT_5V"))
 (segment (start 40.3 37.2) (end 39.5983 37.2) (width 0.2) (layer "F.Cu") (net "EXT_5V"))
 (segment (start 47.15 37.2) (end 46.5483 37.2) (width 0.2) (layer "F.Cu") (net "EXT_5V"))
 (segment (start 40.4247 38.1017) (end 39.5983 37.2753) (width 0.2) (layer "F.Cu") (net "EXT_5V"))
 (segment (start 45.6466 38.1017) (end 40.4247 38.1017) (width 0.2) (layer "F.Cu") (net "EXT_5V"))
 (segment (start 34.35 37.8017) (end 37.55 37.8017) (width 0.2) (layer "F.Cu") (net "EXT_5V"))
 (segment (start 37.05 28.6999) (end 37.05 27.7982) (width 0.2) (layer "F.Cu") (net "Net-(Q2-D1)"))
 (segment (start 37.2177 32.7759) (end 37.4401 32.9983) (width 0.2) (layer "F.Cu") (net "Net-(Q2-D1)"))
 (segment (start 37.55 33.6) (end 37.55 32.9983) (width 0.2) (layer "F.Cu") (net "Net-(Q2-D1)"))
 (segment (start 37.4401 32.9983) (end 37.55 32.9983) (width 0.2) (layer "F.Cu") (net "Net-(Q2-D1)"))
 (segment (start 37.05 27.7982) (end 36.3666 27.7982) (width 0.2) (layer "F.Cu") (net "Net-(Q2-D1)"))
 (via (at 37.2177 32.7759) (size 0.6) (drill 0.3) (layers "F.Cu" "B.Cu") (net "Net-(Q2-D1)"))
 (via (at 36.3666 27.7982) (size 0.6) (drill 0.3) (layers "F.Cu" "B.Cu") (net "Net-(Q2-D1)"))
 (segment (start 37.2177 28.6493) (end 36.3666 27.7982) (width 0.2) (layer "B.Cu") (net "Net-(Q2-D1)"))
 (segment (start 37.2177 32.7759) (end 37.2177 28.6493) (width 0.2) (layer "B.Cu") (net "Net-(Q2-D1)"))
 (segment (start 46.6983 34.65) (end 45.7966 35.5517) (width 0.2) (layer "F.Cu") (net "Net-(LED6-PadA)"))
 (segment (start 45.7966 35.5517) (end 37.5 35.5517) (width 0.2) (layer "F.Cu") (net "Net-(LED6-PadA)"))
 (segment (start 35.25 37.2) (end 35.8517 37.2) (width 0.2) (layer "F.Cu") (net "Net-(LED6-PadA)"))
 (segment (start 37.5 35.5517) (end 35.8517 37.2) (width 0.2) (layer "F.Cu") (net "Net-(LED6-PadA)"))
 (segment (start 47.6 34.65) (end 46.6983 34.65) (width 0.2) (layer "F.Cu") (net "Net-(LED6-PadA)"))
 (segment (start 40.75 30) (end 40.1483 30) (width 0.2) (layer "F.Cu") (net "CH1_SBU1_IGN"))
 (segment (start 30.4583 32.9983) (end 35.25 32.9983) (width 0.2) (layer "F.Cu") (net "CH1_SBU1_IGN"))
 (segment (start 37.05 31.3001) (end 35.3503 32.9998) (width 0.2) (layer "F.Cu") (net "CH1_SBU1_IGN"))
 (segment (start 35.25 32.9998) (end 35.25 32.9983) (width 0.2) (layer "F.Cu") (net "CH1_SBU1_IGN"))
 (segment (start 40.145 29.9967) (end 37.4517 29.9967) (width 0.2) (layer "F.Cu") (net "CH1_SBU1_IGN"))
 (segment (start 40.1483 30) (end 40.145 29.9967) (width 0.2) (layer "F.Cu") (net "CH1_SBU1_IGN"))
 (segment (start 35.25 33.6) (end 35.25 32.9998) (width 0.2) (layer "F.Cu") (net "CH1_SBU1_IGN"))
 (segment (start 37.05 31.3001) (end 37.05 30.3984) (width 0.2) (layer "F.Cu") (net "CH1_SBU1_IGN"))
 (segment (start 28.73 31.27) (end 30.4583 32.9983) (width 0.2) (layer "F.Cu") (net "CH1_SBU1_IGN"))
 (segment (start 35.3503 32.9998) (end 35.25 32.9998) (width 0.2) (layer "F.Cu") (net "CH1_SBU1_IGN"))
 (segment (start 37.4517 29.9967) (end 37.05 30.3984) (width 0.2) (layer "F.Cu") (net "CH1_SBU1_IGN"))
 (segment (start 43.1102 36.9619) (end 43.012 36.9619) (width 0.2) (layer "F.Cu") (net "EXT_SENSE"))
 (segment (start 43.3483 37.2) (end 43.1102 36.9619) (width 0.2) (layer "F.Cu") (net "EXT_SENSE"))
 (segment (start 43.95 37.2) (end 43.3483 37.2) (width 0.2) (layer "F.Cu") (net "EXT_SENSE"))
 (via (at 43.012 36.9619) (size 0.6) (drill 0.3) (layers "F.Cu" "B.Cu") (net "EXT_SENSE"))
 (segment (start 40.5527 36.9619) (end 35.2102 31.6194) (width 0.2) (layer "B.Cu") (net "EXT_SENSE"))
 (segment (start 32.54 30) (end 31.27 28.73) (width 0.2) (layer "B.Cu") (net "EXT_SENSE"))
 (segment (start 35.2102 30.894) (end 34.3162 30) (width 0.2) (layer "B.Cu") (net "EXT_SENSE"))
 (segment (start 34.3162 30) (end 32.54 30) (width 0.2) (layer "B.Cu") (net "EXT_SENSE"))
 (segment (start 43.012 36.9619) (end 40.5527 36.9619) (width 0.2) (layer "B.Cu") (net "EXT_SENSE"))
 (segment (start 35.2102 31.6194) (end 35.2102 30.894) (width 0.2) (layer "B.Cu") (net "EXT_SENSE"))
 (segment (start 43.45 34.6) (end 42.7483 34.6) (width 0.2) (layer "F.Cu") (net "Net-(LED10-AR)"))
 (segment (start 42.6652 34.6831) (end 42.7483 34.6) (width 0.2) (layer "F.Cu") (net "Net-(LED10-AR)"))
 (segment (start 34.35 34.2017) (end 34.8314 34.6831) (width 0.2) (layer "F.Cu") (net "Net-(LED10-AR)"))
 (segment (start 34.35 33.6) (end 34.35 34.2017) (width 0.2) (layer "F.Cu") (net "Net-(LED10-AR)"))
 (segment (start 34.8314 34.6831) (end 42.6652 34.6831) (width 0.2) (layer "F.Cu") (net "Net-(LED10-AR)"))
 (segment (start 45.35 34.6) (end 44.6483 34.6) (width 0.2) (layer "F.Cu") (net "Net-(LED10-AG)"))
 (segment (start 47.15 29.3983) (end 48.5133 29.3983) (width 0.2) (layer "F.Cu") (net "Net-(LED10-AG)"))
 (segment (start 45.393 31.6483) (end 45.3069 31.7344) (width 0.2) (layer "F.Cu") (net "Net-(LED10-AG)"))
 (segment (start 47.6258 31.6483) (end 45.393 31.6483) (width 0.2) (layer "F.Cu") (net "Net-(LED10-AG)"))
 (segment (start 43.6484 33.1486) (end 44.6483 34.1485) (width 0.2) (layer "F.Cu") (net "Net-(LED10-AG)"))
 (segment (start 45.3069 31.7344) (end 43.8231 31.7344) (width 0.2) (layer "F.Cu") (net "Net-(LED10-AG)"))
 (segment (start 48.6661 29.5511) (end 48.6661 30.608) (width 0.2) (layer "F.Cu") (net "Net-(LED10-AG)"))
 (segment (start 48.6661 30.608) (end 47.6258 31.6483) (width 0.2) (layer "F.Cu") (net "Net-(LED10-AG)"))
 (segment (start 43.6484 31.9091) (end 43.6484 33.1486) (width 0.2) (layer "F.Cu") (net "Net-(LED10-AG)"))
 (segment (start 47.15 30) (end 47.15 29.3983) (width 0.2) (layer "F.Cu") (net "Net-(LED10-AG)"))
 (segment (start 43.8231 31.7344) (end 43.6484 31.9091) (width 0.2) (layer "F.Cu") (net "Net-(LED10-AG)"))
 (segment (start 48.5133 29.3983) (end 48.6661 29.5511) (width 0.2) (layer "F.Cu") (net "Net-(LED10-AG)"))
 (segment (start 44.6483 34.1485) (end 44.6483 34.6) (width 0.2) (layer "F.Cu") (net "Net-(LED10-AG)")))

